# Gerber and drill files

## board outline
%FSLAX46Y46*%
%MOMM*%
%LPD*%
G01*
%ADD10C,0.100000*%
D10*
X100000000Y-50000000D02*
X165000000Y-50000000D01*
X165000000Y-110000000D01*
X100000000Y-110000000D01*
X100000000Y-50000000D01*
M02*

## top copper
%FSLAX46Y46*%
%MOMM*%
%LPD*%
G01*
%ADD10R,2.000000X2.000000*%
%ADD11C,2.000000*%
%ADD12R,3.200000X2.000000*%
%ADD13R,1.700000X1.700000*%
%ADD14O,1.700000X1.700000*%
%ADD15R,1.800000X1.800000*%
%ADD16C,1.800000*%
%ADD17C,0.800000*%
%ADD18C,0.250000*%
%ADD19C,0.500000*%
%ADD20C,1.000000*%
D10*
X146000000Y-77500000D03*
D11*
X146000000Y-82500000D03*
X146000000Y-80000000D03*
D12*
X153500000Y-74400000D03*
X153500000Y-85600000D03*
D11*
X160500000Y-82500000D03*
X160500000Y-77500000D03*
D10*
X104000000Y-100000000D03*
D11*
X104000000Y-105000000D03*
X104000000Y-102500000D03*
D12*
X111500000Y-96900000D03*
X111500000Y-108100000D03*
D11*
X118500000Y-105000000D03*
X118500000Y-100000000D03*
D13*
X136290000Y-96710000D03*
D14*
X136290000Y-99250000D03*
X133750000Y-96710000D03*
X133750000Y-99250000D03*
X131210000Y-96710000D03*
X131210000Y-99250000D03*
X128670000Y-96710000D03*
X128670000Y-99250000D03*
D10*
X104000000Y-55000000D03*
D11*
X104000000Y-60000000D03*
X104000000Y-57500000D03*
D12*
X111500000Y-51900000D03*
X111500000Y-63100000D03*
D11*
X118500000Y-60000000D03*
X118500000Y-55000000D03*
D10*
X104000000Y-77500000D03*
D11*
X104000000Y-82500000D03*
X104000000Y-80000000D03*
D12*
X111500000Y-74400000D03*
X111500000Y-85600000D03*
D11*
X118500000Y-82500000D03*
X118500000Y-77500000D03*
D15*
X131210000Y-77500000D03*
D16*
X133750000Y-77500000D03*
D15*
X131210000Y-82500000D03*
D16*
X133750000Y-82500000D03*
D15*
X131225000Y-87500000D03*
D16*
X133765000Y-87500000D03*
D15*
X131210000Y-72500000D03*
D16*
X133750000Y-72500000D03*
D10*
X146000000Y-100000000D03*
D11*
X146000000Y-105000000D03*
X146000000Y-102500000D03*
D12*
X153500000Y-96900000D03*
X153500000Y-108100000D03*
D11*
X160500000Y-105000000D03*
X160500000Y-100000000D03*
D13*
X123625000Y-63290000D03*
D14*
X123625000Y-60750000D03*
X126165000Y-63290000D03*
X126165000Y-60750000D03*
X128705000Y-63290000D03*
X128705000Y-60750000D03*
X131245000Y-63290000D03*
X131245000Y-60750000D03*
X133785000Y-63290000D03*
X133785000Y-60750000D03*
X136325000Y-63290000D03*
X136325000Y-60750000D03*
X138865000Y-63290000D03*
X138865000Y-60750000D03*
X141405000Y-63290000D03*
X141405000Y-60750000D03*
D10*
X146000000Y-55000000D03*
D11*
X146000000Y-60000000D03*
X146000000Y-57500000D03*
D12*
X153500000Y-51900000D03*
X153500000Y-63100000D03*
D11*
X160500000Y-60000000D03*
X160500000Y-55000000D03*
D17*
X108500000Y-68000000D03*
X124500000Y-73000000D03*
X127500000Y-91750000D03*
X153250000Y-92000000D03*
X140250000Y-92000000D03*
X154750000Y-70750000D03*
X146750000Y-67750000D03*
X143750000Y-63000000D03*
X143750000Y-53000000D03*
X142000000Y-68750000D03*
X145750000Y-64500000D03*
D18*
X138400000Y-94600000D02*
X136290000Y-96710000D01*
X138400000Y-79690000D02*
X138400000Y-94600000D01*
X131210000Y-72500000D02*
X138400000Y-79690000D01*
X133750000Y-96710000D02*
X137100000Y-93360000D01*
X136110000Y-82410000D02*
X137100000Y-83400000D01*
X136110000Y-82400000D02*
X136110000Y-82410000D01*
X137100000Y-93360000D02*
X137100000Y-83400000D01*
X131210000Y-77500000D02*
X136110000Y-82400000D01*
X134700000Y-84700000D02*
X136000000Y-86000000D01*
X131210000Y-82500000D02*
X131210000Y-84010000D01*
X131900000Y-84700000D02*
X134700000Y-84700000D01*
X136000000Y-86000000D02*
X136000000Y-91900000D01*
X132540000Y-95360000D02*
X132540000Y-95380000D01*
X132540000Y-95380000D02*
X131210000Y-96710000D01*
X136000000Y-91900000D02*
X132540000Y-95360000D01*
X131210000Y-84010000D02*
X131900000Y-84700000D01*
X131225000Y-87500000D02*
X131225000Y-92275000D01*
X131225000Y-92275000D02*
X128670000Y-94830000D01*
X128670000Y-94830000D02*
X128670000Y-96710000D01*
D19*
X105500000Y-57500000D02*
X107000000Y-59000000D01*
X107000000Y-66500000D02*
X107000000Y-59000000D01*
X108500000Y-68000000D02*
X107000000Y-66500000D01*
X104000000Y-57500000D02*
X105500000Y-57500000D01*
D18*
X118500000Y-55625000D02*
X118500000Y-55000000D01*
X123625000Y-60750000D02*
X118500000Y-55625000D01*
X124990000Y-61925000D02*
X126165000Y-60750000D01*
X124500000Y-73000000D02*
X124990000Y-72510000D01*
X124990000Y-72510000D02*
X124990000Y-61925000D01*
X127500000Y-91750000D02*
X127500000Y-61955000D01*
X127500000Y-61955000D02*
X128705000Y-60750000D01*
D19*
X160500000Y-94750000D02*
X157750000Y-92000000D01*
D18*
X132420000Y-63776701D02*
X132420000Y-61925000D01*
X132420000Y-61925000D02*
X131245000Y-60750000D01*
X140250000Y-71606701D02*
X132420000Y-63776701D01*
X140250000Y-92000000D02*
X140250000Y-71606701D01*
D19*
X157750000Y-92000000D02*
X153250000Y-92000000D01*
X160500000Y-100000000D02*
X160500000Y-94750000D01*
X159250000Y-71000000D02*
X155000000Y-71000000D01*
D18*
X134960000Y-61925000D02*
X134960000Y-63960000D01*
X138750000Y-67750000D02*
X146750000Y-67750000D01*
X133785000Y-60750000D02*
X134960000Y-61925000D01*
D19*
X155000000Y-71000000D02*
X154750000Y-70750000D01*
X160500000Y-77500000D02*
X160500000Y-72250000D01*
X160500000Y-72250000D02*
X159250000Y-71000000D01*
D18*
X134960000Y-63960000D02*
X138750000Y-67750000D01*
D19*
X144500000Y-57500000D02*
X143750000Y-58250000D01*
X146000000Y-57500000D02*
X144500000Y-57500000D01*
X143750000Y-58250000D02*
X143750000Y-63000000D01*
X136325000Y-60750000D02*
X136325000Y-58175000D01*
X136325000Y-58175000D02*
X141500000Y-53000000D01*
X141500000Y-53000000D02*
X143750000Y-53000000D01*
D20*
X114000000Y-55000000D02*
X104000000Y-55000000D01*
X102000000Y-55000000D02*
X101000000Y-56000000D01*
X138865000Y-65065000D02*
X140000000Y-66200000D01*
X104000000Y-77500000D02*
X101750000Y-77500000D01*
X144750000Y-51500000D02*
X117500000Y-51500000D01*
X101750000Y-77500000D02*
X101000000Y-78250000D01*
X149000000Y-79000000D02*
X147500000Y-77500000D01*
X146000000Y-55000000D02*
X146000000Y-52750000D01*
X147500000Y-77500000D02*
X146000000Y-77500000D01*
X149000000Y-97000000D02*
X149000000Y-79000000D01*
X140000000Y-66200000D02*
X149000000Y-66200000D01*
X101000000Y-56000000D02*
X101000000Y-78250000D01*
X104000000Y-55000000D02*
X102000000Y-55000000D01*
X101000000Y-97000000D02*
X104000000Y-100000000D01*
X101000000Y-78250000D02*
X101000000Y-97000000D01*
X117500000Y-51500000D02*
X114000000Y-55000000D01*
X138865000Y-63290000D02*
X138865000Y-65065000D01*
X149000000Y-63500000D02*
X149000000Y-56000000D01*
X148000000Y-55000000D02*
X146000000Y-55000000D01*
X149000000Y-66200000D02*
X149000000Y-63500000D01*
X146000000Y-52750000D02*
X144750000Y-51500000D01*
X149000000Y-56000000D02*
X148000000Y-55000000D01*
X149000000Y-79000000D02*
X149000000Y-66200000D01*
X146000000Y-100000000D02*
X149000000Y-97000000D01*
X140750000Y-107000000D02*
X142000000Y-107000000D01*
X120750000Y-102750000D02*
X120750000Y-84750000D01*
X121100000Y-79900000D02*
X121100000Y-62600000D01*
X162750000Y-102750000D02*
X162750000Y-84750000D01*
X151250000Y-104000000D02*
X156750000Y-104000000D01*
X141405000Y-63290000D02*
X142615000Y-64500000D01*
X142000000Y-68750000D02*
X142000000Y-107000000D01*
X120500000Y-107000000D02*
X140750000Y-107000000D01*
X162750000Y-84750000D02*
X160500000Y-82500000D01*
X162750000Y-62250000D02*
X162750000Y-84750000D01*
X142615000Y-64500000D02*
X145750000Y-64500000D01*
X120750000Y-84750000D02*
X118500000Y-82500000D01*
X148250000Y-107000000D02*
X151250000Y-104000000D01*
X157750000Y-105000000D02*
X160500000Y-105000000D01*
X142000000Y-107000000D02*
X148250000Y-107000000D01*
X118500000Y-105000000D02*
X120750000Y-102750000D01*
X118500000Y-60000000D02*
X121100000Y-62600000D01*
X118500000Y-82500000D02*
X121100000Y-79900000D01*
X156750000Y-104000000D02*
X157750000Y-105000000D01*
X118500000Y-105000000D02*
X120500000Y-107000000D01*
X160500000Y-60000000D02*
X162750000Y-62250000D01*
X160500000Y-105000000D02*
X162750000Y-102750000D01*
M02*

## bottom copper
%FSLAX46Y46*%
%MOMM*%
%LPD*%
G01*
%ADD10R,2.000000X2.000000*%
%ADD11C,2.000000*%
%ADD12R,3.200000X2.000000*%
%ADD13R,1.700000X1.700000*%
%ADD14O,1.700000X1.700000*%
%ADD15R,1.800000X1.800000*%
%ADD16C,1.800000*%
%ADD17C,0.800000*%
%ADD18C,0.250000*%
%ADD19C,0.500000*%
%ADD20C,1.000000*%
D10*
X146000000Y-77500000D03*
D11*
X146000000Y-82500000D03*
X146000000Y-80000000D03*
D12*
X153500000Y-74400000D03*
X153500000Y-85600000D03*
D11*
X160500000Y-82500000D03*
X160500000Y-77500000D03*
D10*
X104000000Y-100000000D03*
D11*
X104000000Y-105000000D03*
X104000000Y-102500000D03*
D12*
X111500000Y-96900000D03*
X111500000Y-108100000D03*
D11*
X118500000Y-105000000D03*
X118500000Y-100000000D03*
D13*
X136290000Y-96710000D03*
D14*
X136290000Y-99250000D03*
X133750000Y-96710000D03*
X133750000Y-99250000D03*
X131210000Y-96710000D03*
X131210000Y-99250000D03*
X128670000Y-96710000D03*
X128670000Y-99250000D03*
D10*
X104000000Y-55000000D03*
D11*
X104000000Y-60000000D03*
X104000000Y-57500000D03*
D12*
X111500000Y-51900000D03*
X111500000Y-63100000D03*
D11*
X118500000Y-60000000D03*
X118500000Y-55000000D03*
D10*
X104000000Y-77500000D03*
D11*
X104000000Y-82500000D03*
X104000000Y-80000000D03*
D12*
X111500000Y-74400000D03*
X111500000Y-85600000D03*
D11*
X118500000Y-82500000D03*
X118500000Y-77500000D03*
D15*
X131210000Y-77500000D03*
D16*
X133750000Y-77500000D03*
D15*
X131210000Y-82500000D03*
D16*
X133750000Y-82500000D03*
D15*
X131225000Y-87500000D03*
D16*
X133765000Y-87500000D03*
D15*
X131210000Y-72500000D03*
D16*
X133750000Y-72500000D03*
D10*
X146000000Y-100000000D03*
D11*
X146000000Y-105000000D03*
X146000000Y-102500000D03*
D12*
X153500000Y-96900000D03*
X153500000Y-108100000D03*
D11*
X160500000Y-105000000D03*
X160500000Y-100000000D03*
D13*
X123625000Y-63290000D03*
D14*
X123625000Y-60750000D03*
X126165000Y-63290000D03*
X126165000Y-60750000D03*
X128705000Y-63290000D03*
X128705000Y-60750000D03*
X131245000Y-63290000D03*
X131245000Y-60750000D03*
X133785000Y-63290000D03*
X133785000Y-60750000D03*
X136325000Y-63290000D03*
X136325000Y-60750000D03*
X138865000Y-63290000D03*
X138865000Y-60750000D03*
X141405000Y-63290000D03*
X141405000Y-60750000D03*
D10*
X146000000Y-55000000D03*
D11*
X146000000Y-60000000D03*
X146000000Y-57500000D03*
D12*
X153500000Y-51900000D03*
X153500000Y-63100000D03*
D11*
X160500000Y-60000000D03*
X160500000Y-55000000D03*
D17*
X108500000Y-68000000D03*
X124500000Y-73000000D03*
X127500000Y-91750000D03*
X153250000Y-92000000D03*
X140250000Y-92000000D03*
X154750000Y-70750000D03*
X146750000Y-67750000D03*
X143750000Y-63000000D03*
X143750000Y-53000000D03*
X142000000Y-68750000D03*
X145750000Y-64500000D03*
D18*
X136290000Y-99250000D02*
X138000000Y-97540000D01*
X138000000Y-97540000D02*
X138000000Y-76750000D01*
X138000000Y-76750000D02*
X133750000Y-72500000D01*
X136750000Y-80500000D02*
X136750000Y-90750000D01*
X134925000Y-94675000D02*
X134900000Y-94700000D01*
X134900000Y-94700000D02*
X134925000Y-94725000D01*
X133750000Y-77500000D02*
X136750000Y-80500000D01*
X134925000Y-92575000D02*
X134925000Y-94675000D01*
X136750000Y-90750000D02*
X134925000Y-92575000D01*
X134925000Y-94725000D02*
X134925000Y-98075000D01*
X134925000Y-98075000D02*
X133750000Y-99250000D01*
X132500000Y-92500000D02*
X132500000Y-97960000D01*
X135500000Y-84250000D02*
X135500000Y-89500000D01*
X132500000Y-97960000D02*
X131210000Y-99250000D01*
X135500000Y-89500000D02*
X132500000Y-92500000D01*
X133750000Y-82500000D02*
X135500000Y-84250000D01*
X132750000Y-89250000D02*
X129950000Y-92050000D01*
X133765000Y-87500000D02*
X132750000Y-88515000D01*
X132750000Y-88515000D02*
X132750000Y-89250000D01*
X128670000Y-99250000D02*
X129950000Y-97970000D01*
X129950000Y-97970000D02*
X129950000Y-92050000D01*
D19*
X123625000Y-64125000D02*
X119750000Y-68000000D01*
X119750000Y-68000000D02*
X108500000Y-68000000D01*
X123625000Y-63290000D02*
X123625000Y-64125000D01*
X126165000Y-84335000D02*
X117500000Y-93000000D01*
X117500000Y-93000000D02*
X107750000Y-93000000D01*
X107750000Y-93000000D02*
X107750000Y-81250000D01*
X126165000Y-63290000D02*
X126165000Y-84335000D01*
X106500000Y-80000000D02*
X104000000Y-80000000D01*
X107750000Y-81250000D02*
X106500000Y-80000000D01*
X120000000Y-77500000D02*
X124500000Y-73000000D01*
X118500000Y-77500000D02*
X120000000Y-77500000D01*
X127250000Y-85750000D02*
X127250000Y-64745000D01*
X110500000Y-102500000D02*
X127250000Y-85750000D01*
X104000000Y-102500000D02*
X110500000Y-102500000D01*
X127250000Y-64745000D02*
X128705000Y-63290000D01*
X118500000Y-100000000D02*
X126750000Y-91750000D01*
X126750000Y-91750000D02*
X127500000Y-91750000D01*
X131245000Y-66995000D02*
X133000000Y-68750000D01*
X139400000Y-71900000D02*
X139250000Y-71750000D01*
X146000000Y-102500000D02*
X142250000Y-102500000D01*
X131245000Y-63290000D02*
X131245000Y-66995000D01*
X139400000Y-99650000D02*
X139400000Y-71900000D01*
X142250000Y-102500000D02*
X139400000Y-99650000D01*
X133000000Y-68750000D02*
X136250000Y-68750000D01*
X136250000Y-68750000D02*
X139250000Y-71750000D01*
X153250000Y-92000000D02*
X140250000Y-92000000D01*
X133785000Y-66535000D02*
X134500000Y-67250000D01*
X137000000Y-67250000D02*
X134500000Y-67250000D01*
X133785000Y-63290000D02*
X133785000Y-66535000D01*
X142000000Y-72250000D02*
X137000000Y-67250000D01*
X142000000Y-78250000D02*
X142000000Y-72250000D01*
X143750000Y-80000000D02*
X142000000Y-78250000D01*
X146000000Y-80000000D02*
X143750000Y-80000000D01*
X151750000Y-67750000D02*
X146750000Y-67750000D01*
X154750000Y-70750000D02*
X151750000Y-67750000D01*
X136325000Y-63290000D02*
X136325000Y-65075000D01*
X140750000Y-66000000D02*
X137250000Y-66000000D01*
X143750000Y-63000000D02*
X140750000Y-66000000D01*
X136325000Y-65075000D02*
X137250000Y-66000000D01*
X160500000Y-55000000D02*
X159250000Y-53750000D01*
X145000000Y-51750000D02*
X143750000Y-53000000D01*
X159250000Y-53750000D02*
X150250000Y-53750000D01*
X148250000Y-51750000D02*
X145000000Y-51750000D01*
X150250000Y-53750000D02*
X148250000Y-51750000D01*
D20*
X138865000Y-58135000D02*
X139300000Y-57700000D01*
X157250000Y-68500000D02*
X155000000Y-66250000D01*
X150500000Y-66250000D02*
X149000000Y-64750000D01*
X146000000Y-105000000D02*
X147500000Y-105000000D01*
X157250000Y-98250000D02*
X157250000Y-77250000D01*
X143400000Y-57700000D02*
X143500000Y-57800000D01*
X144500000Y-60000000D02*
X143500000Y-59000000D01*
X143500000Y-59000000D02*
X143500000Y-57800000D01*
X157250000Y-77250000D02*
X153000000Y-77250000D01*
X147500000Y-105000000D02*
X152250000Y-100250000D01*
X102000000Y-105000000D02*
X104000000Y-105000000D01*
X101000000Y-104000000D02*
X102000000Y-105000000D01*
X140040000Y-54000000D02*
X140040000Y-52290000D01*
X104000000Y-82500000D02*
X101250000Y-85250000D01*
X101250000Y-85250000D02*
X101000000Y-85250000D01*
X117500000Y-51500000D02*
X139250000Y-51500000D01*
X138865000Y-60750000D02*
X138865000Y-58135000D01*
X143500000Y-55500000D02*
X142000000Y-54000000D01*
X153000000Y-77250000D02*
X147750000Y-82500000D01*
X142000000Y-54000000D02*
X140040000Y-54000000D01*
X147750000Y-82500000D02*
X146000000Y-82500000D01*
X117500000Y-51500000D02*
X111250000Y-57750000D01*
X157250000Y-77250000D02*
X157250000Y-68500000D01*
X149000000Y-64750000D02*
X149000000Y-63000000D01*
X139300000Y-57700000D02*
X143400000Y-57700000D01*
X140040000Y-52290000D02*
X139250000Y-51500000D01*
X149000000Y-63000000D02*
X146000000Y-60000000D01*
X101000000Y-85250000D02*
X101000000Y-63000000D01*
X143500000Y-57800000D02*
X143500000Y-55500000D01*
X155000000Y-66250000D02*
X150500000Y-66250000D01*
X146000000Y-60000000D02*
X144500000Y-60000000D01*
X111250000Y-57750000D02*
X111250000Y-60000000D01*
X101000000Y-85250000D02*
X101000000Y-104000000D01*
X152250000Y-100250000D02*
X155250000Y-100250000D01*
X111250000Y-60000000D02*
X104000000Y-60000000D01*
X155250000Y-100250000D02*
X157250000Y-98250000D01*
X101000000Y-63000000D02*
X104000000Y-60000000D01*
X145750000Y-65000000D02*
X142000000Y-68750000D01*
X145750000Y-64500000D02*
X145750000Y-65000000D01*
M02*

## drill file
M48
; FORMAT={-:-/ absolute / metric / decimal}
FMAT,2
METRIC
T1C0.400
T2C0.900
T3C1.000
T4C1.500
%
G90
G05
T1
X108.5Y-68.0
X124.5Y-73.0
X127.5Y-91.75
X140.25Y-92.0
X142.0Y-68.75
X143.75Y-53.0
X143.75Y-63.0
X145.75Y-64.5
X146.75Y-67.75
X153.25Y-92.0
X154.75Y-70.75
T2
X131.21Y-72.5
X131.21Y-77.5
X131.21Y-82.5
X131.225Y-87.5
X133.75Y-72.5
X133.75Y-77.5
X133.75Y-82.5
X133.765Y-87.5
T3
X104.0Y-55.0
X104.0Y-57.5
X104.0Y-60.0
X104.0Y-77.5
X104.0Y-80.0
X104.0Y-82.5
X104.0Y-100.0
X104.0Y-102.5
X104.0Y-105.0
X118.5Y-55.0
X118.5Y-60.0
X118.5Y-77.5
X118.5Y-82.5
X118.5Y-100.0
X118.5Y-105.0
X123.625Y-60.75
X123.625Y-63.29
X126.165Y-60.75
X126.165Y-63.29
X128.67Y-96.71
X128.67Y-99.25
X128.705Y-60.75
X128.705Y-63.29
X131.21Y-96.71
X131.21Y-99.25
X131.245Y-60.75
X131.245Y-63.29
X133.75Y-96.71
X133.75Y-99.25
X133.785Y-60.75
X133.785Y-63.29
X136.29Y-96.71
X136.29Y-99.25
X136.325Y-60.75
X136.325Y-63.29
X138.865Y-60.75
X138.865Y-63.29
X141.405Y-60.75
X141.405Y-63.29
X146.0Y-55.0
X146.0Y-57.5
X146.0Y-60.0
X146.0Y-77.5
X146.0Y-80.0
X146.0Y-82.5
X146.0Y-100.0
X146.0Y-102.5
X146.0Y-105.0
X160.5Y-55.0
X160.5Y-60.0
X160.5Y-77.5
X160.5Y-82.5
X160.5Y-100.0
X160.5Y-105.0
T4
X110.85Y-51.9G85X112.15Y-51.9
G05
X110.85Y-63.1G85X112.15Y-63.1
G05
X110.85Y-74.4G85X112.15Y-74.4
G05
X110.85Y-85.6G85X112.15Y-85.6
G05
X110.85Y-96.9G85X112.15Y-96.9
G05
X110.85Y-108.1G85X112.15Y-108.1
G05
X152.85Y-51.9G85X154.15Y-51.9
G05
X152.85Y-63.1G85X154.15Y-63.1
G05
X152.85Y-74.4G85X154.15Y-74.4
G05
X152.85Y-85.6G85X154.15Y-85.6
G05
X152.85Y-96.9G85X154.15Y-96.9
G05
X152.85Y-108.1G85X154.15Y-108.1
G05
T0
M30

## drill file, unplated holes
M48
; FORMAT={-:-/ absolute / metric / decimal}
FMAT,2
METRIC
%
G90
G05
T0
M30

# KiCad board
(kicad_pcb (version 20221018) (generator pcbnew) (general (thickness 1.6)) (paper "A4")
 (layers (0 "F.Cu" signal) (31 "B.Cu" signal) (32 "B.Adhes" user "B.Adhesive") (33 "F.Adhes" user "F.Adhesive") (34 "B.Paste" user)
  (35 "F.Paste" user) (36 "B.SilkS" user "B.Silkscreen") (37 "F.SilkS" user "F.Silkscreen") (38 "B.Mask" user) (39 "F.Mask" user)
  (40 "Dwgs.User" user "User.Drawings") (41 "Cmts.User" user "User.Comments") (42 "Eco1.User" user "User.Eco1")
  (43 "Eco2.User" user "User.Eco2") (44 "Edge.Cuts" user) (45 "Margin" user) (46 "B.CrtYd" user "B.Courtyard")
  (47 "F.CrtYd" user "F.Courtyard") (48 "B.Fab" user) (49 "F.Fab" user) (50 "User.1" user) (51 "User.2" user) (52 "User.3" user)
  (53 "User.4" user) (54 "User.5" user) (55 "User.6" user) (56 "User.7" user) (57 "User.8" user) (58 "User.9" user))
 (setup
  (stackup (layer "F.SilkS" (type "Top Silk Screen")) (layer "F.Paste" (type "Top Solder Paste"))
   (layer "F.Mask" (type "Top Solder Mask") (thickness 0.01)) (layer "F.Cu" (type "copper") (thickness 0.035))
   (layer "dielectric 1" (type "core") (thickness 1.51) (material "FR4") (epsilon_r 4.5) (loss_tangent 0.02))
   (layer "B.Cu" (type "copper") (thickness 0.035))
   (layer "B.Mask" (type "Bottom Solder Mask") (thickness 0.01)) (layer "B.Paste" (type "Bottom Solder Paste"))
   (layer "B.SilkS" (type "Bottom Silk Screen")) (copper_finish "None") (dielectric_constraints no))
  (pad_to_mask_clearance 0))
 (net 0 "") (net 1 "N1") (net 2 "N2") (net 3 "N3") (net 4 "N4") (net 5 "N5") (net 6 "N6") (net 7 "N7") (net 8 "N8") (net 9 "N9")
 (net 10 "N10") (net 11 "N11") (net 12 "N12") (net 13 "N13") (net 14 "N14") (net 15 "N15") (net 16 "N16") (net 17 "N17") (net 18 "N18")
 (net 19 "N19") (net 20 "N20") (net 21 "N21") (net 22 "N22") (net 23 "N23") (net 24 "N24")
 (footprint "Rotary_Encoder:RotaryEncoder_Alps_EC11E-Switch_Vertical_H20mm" (layer "F.Cu") (at 146 77.5)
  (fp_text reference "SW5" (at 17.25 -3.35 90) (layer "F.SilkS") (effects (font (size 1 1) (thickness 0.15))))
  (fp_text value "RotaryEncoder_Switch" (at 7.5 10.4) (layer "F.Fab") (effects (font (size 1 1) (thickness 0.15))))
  (pad "A" thru_hole rect (at 0 0) (size 2 2) (drill 1) (layers "*.Cu" "*.Mask") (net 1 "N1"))
  (pad "B" thru_hole circle (at 0 5) (size 2 2) (drill 1) (layers "*.Cu" "*.Mask") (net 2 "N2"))
  (pad "C" thru_hole circle (at 0 2.5) (size 2 2) (drill 1) (layers "*.Cu" "*.Mask") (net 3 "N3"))
  (pad "MP" thru_hole rect (at 7.5 -3.1) (size 3.2 2) (drill oval 2.8 1.5) (layers "*.Cu" "*.Mask"))
  (pad "MP" thru_hole rect (at 7.5 8.1) (size 3.2 2) (drill oval 2.8 1.5) (layers "*.Cu" "*.Mask"))
  (pad "S1" thru_hole circle (at 14.5 5) (size 2 2) (drill 1) (layers "*.Cu" "*.Mask") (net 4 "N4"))
  (pad "S2" thru_hole circle (at 14.5 0) (size 2 2) (drill 1) (layers "*.Cu" "*.Mask") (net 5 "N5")))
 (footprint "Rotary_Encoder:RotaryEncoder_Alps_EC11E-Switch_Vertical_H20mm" (layer "F.Cu") (at 104 100)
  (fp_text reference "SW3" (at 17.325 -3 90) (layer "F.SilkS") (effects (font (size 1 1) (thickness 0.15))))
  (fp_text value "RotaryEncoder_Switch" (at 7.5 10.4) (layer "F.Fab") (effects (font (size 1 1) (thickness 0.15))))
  (pad "A" thru_hole rect (at 0 0) (size 2 2) (drill 1) (layers "*.Cu" "*.Mask") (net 1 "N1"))
  (pad "B" thru_hole circle (at 0 5) (size 2 2) (drill 1) (layers "*.Cu" "*.Mask") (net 2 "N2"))
  (pad "C" thru_hole circle (at 0 2.5) (size 2 2) (drill 1) (layers "*.Cu" "*.Mask") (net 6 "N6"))
  (pad "MP" thru_hole rect (at 7.5 -3.1) (size 3.2 2) (drill oval 2.8 1.5) (layers "*.Cu" "*.Mask"))
  (pad "MP" thru_hole rect (at 7.5 8.1) (size 3.2 2) (drill oval 2.8 1.5) (layers "*.Cu" "*.Mask"))
  (pad "S1" thru_hole circle (at 14.5 5) (size 2 2) (drill 1) (layers "*.Cu" "*.Mask") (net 4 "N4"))
  (pad "S2" thru_hole circle (at 14.5 0) (size 2 2) (drill 1) (layers "*.Cu" "*.Mask") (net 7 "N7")))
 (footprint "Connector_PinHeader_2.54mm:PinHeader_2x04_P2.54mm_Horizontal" (layer "F.Cu") (at 136.29 96.71 -90)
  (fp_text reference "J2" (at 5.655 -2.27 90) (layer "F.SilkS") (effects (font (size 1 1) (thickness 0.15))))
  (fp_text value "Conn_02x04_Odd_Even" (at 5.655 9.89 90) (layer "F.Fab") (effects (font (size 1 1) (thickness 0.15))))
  (pad "1" thru_hole rect (at 0 0 270) (size 1.7 1.7) (drill 1) (layers "*.Cu" "*.Mask") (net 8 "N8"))
  (pad "2" thru_hole oval (at 2.54 0 270) (size 1.7 1.7) (drill 1) (layers "*.Cu" "*.Mask") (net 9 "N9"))
  (pad "3" thru_hole oval (at 0 2.54 270) (size 1.7 1.7) (drill 1) (layers "*.Cu" "*.Mask") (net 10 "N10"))
  (pad "4" thru_hole oval (at 2.54 2.54 270) (size 1.7 1.7) (drill 1) (layers "*.Cu" "*.Mask") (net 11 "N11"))
  (pad "5" thru_hole oval (at 0 5.08 270) (size 1.7 1.7) (drill 1) (layers "*.Cu" "*.Mask") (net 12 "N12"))
  (pad "6" thru_hole oval (at 2.54 5.08 270) (size 1.7 1.7) (drill 1) (layers "*.Cu" "*.Mask") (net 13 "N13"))
  (pad "7" thru_hole oval (at 0 7.62 270) (size 1.7 1.7) (drill 1) (layers "*.Cu" "*.Mask") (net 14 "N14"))
  (pad "8" thru_hole oval (at 2.54 7.62 270) (size 1.7 1.7) (drill 1) (layers "*.Cu" "*.Mask") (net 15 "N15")))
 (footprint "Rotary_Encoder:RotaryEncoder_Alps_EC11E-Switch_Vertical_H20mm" (layer "F.Cu") (at 104 55)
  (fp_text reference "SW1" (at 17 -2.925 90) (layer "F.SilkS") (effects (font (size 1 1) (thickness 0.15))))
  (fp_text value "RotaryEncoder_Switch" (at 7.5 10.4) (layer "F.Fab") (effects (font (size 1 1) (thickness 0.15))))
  (pad "A" thru_hole rect (at 0 0) (size 2 2) (drill 1) (layers "*.Cu" "*.Mask") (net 1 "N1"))
  (pad "B" thru_hole circle (at 0 5) (size 2 2) (drill 1) (layers "*.Cu" "*.Mask") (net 2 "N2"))
  (pad "C" thru_hole circle (at 0 2.5) (size 2 2) (drill 1) (layers "*.Cu" "*.Mask") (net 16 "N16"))
  (pad "MP" thru_hole rect (at 7.5 -3.1) (size 3.2 2) (drill oval 2.8 1.5) (layers "*.Cu" "*.Mask"))
  (pad "MP" thru_hole rect (at 7.5 8.1) (size 3.2 2) (drill oval 2.8 1.5) (layers "*.Cu" "*.Mask"))
  (pad "S1" thru_hole circle (at 14.5 5) (size 2 2) (drill 1) (layers "*.Cu" "*.Mask") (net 4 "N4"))
  (pad "S2" thru_hole circle (at 14.5 0) (size 2 2) (drill 1) (layers "*.Cu" "*.Mask") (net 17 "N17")))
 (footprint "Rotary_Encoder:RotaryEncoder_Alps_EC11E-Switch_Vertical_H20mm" (layer "F.Cu") (at 104 77.5)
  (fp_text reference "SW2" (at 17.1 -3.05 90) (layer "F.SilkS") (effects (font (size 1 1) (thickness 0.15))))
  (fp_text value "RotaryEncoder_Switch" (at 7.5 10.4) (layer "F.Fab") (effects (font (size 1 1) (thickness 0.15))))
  (pad "A" thru_hole rect (at 0 0) (size 2 2) (drill 1) (layers "*.Cu" "*.Mask") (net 1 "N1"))
  (pad "B" thru_hole circle (at 0 5) (size 2 2) (drill 1) (layers "*.Cu" "*.Mask") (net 2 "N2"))
  (pad "C" thru_hole circle (at 0 2.5) (size 2 2) (drill 1) (layers "*.Cu" "*.Mask") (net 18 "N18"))
  (pad "MP" thru_hole rect (at 7.5 -3.1) (size 3.2 2) (drill oval 2.8 1.5) (layers "*.Cu" "*.Mask"))
  (pad "MP" thru_hole rect (at 7.5 8.1) (size 3.2 2) (drill oval 2.8 1.5) (layers "*.Cu" "*.Mask"))
  (pad "S1" thru_hole circle (at 14.5 5) (size 2 2) (drill 1) (layers "*.Cu" "*.Mask") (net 4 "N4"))
  (pad "S2" thru_hole circle (at 14.5 0) (size 2 2) (drill 1) (layers "*.Cu" "*.Mask") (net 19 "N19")))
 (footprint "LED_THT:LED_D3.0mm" (layer "F.Cu") (at 131.21 77.5)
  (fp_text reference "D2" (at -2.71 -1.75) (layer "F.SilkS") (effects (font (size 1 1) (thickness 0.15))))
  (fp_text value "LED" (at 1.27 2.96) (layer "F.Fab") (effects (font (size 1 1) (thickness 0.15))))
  (pad "1" thru_hole rect (at 0 0) (size 1.8 1.8) (drill 0.9) (layers "*.Cu" "*.Mask") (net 10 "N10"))
  (pad "2" thru_hole circle (at 2.54 0) (size 1.8 1.8) (drill 0.9) (layers "*.Cu" "*.Mask") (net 11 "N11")))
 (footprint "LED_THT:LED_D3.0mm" (layer "F.Cu") (at 131.21 82.5)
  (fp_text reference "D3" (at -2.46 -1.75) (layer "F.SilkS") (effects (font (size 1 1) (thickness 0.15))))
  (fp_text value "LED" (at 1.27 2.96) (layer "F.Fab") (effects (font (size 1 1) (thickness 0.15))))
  (pad "1" thru_hole rect (at 0 0) (size 1.8 1.8) (drill 0.9) (layers "*.Cu" "*.Mask") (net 12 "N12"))
  (pad "2" thru_hole circle (at 2.54 0) (size 1.8 1.8) (drill 0.9) (layers "*.Cu" "*.Mask") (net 13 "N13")))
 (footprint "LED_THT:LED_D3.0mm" (layer "F.Cu") (at 131.225 87.5)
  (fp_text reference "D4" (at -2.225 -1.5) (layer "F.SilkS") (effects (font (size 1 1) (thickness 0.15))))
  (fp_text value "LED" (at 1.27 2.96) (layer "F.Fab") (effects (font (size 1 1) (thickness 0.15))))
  (pad "1" thru_hole rect (at 0 0) (size 1.8 1.8) (drill 0.9) (layers "*.Cu" "*.Mask") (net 14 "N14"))
  (pad "2" thru_hole circle (at 2.54 0) (size 1.8 1.8) (drill 0.9) (layers "*.Cu" "*.Mask") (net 15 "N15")))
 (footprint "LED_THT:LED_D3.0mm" (layer "F.Cu") (at 131.21 72.5)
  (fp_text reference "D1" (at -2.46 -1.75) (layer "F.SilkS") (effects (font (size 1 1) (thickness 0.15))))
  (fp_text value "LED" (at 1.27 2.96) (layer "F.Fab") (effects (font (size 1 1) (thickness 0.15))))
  (pad "1" thru_hole rect (at 0 0) (size 1.8 1.8) (drill 0.9) (layers "*.Cu" "*.Mask") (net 8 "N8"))
  (pad "2" thru_hole circle (at 2.54 0) (size 1.8 1.8) (drill 0.9) (layers "*.Cu" "*.Mask") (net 9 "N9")))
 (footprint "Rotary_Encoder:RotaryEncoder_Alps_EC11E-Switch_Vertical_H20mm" (layer "F.Cu") (at 146 100)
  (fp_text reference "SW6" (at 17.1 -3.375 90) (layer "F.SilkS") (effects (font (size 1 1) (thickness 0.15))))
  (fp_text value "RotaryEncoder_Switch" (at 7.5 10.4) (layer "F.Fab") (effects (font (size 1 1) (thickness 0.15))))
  (pad "A" thru_hole rect (at 0 0) (size 2 2) (drill 1) (layers "*.Cu" "*.Mask") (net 1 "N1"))
  (pad "B" thru_hole circle (at 0 5) (size 2 2) (drill 1) (layers "*.Cu" "*.Mask") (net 2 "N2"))
  (pad "C" thru_hole circle (at 0 2.5) (size 2 2) (drill 1) (layers "*.Cu" "*.Mask") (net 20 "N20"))
  (pad "MP" thru_hole rect (at 7.5 -3.1) (size 3.2 2) (drill oval 2.8 1.5) (layers "*.Cu" "*.Mask"))
  (pad "MP" thru_hole rect (at 7.5 8.1) (size 3.2 2) (drill oval 2.8 1.5) (layers "*.Cu" "*.Mask"))
  (pad "S1" thru_hole circle (at 14.5 5) (size 2 2) (drill 1) (layers "*.Cu" "*.Mask") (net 4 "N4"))
  (pad "S2" thru_hole circle (at 14.5 0) (size 2 2) (drill 1) (layers "*.Cu" "*.Mask") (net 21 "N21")))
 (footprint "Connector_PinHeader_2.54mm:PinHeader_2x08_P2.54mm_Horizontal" (layer "F.Cu") (at 123.625 63.29 90)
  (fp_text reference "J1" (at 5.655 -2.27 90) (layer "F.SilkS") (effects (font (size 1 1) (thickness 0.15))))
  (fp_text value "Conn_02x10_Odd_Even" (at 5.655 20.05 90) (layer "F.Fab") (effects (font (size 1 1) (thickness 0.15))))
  (pad "1" thru_hole rect (at 0 0 90) (size 1.7 1.7) (drill 1) (layers "*.Cu" "*.Mask") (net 16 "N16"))
  (pad "2" thru_hole oval (at 2.54 0 90) (size 1.7 1.7) (drill 1) (layers "*.Cu" "*.Mask") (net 17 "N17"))
  (pad "3" thru_hole oval (at 0 2.54 90) (size 1.7 1.7) (drill 1) (layers "*.Cu" "*.Mask") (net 18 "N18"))
  (pad "4" thru_hole oval (at 2.54 2.54 90) (size 1.7 1.7) (drill 1) (layers "*.Cu" "*.Mask") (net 19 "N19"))
  (pad "5" thru_hole oval (at 0 5.08 90) (size 1.7 1.7) (drill 1) (layers "*.Cu" "*.Mask") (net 6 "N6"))
  (pad "6" thru_hole oval (at 2.54 5.08 90) (size 1.7 1.7) (drill 1) (layers "*.Cu" "*.Mask") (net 7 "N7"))
  (pad "7" thru_hole oval (at 0 7.62 90) (size 1.7 1.7) (drill 1) (layers "*.Cu" "*.Mask") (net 20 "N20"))
  (pad "8" thru_hole oval (at 2.54 7.62 90) (size 1.7 1.7) (drill 1) (layers "*.Cu" "*.Mask") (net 21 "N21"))
  (pad "9" thru_hole oval (at 0 10.16 90) (size 1.7 1.7) (drill 1) (layers "*.Cu" "*.Mask") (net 3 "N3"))
  (pad "10" thru_hole oval (at 2.54 10.16 90) (size 1.7 1.7) (drill 1) (layers "*.Cu" "*.Mask") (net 5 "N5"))
  (pad "11" thru_hole oval (at 0 12.7 90) (size 1.7 1.7) (drill 1) (layers "*.Cu" "*.Mask") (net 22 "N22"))
  (pad "12" thru_hole oval (at 2.54 12.7 90) (size 1.7 1.7) (drill 1) (layers "*.Cu" "*.Mask") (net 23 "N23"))
  (pad "13" thru_hole oval (at 0 15.24 90) (size 1.7 1.7) (drill 1) (layers "*.Cu" "*.Mask") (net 1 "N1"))
  (pad "14" thru_hole oval (at 2.54 15.24 90) (size 1.7 1.7) (drill 1) (layers "*.Cu" "*.Mask") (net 2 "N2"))
  (pad "15" thru_hole oval (at 0 17.78 90) (size 1.7 1.7) (drill 1) (layers "*.Cu" "*.Mask") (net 4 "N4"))
  (pad "16" thru_hole oval (at 2.54 17.78 90) (size 1.7 1.7) (drill 1) (layers "*.Cu" "*.Mask") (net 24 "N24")))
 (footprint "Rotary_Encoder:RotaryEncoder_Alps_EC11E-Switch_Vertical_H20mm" (layer "F.Cu") (at 146 55)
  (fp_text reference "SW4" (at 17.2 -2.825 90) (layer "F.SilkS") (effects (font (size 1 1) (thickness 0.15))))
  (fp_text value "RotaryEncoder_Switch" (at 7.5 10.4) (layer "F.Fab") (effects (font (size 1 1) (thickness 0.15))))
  (pad "A" thru_hole rect (at 0 0) (size 2 2) (drill 1) (layers "*.Cu" "*.Mask") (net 1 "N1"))
  (pad "B" thru_hole circle (at 0 5) (size 2 2) (drill 1) (layers "*.Cu" "*.Mask") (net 2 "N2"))
  (pad "C" thru_hole circle (at 0 2.5) (size 2 2) (drill 1) (layers "*.Cu" "*.Mask") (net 22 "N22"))
  (pad "MP" thru_hole rect (at 7.5 -3.1) (size 3.2 2) (drill oval 2.8 1.5) (layers "*.Cu" "*.Mask"))
  (pad "MP" thru_hole rect (at 7.5 8.1) (size 3.2 2) (drill oval 2.8 1.5) (layers "*.Cu" "*.Mask"))
  (pad "S1" thru_hole circle (at 14.5 5) (size 2 2) (drill 1) (layers "*.Cu" "*.Mask") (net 4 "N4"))
  (pad "S2" thru_hole circle (at 14.5 0) (size 2 2) (drill 1) (layers "*.Cu" "*.Mask") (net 23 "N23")))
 (gr_rect (start 100 50) (end 165 110) (stroke (width 0.1) (type default)) (fill none) (layer "Edge.Cuts"))
 (segment (start 138.4 94.6) (end 136.29 96.71) (width 0.25) (layer "F.Cu") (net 8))
 (segment (start 138.4 79.69) (end 138.4 94.6) (width 0.25) (layer "F.Cu") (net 8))
 (segment (start 131.21 72.5) (end 138.4 79.69) (width 0.25) (layer "F.Cu") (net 8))
 (segment (start 136.29 99.25) (end 138 97.54) (width 0.25) (layer "B.Cu") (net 9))
 (segment (start 138 97.54) (end 138 76.75) (width 0.25) (layer "B.Cu") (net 9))
 (segment (start 138 76.75) (end 133.75 72.5) (width 0.25) (layer "B.Cu") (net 9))
 (segment (start 133.75 96.71) (end 137.1 93.36) (width 0.25) (layer "F.Cu") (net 10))
 (segment (start 136.11 82.41) (end 137.1 83.4) (width 0.25) (layer "F.Cu") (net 10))
 (segment (start 136.11 82.4) (end 136.11 82.41) (width 0.25) (layer "F.Cu") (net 10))
 (segment (start 137.1 93.36) (end 137.1 83.4) (width 0.25) (layer "F.Cu") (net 10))
 (segment (start 131.21 77.5) (end 136.11 82.4) (width 0.25) (layer "F.Cu") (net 10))
 (segment (start 136.75 80.5) (end 136.75 90.75) (width 0.25) (layer "B.Cu") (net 11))
 (segment (start 134.925 94.675) (end 134.9 94.7) (width 0.25) (layer "B.Cu") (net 11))
 (segment (start 134.9 94.7) (end 134.925 94.725) (width 0.25) (layer "B.Cu") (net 11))
 (segment (start 133.75 77.5) (end 136.75 80.5) (width 0.25) (layer "B.Cu") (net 11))
 (segment (start 134.925 92.575) (end 134.925 94.675) (width 0.25) (layer "B.Cu") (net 11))
 (segment (start 136.75 90.75) (end 134.925 92.575) (width 0.25) (layer "B.Cu") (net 11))
 (segment (start 134.925 94.725) (end 134.925 98.075) (width 0.25) (layer "B.Cu") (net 11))
 (segment (start 134.925 98.075) (end 133.75 99.25) (width 0.25) (layer "B.Cu") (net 11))
 (segment (start 134.7 84.7) (end 136 86) (width 0.25) (layer "F.Cu") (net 12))
 (segment (start 131.21 82.5) (end 131.21 84.01) (width 0.25) (layer "F.Cu") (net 12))
 (segment (start 131.9 84.7) (end 134.7 84.7) (width 0.25) (layer "F.Cu") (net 12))
 (segment (start 136 86) (end 136 91.9) (width 0.25) (layer "F.Cu") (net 12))
 (segment (start 132.54 95.36) (end 132.54 95.38) (width 0.25) (layer "F.Cu") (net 12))
 (segment (start 132.54 95.38) (end 131.21 96.71) (width 0.25) (layer "F.Cu") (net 12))
 (segment (start 136 91.9) (end 132.54 95.36) (width 0.25) (layer "F.Cu") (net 12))
 (segment (start 131.21 84.01) (end 131.9 84.7) (width 0.25) (layer "F.Cu") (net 12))
 (segment (start 132.5 92.5) (end 132.5 97.96) (width 0.25) (layer "B.Cu") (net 13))
 (segment (start 135.5 84.25) (end 135.5 89.5) (width 0.25) (layer "B.Cu") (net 13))
 (segment (start 132.5 97.96) (end 131.21 99.25) (width 0.25) (layer "B.Cu") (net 13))
 (segment (start 135.5 89.5) (end 132.5 92.5) (width 0.25) (layer "B.Cu") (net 13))
 (segment (start 133.75 82.5) (end 135.5 84.25) (width 0.25) (layer "B.Cu") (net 13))
 (segment (start 131.225 87.5) (end 131.225 92.275) (width 0.25) (layer "F.Cu") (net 14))
 (segment (start 131.225 92.275) (end 128.67 94.83) (width 0.25) (layer "F.Cu") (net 14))
 (segment (start 128.67 94.83) (end 128.67 96.71) (width 0.25) (layer "F.Cu") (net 14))
 (segment (start 132.75 89.25) (end 129.95 92.05) (width 0.25) (layer "B.Cu") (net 15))
 (segment (start 133.765 87.5) (end 132.75 88.515) (width 0.25) (layer "B.Cu") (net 15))
 (segment (start 132.75 88.515) (end 132.75 89.25) (width 0.25) (layer "B.Cu") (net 15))
 (segment (start 128.67 99.25) (end 129.95 97.97) (width 0.25) (layer "B.Cu") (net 15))
 (segment (start 129.95 97.97) (end 129.95 92.05) (width 0.25) (layer "B.Cu") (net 15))
 (segment (start 105.5 57.5) (end 107 59) (width 0.5) (layer "F.Cu") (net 16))
 (segment (start 107 66.5) (end 107 59) (width 0.5) (layer "F.Cu") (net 16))
 (segment (start 108.5 68) (end 107 66.5) (width 0.5) (layer "F.Cu") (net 16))
 (segment (start 104 57.5) (end 105.5 57.5) (width 0.5) (layer "F.Cu") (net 16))
 (via (at 108.5 68) (size 0.8) (drill 0.4) (layers "F.Cu" "B.Cu") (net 16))
 (segment (start 123.625 64.125) (end 119.75 68) (width 0.5) (layer "B.Cu") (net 16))
 (segment (start 119.75 68) (end 108.5 68) (width 0.5) (layer "B.Cu") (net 16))
 (segment (start 123.625 63.29) (end 123.625 64.125) (width 0.5) (layer "B.Cu") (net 16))
 (segment (start 118.5 55.625) (end 118.5 55) (width 0.25) (layer "F.Cu") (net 17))
 (segment (start 123.625 60.75) (end 118.5 55.625) (width 0.25) (layer "F.Cu") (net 17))
 (segment (start 126.165 84.335) (end 117.5 93) (width 0.5) (layer "B.Cu") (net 18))
 (segment (start 117.5 93) (end 107.75 93) (width 0.5) (layer "B.Cu") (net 18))
 (segment (start 107.75 93) (end 107.75 81.25) (width 0.5) (layer "B.Cu") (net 18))
 (segment (start 126.165 63.29) (end 126.165 84.335) (width 0.5) (layer "B.Cu") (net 18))
 (segment (start 106.5 80) (end 104 80) (width 0.5) (layer "B.Cu") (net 18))
 (segment (start 107.75 81.25) (end 106.5 80) (width 0.5) (layer "B.Cu") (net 18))
 (segment (start 124.99 61.925) (end 126.165 60.75) (width 0.25) (layer "F.Cu") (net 19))
 (segment (start 124.5 73) (end 124.99 72.51) (width 0.25) (layer "F.Cu") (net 19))
 (segment (start 124.99 72.51) (end 124.99 61.925) (width 0.25) (layer "F.Cu") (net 19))
 (via (at 124.5 73) (size 0.8) (drill 0.4) (layers "F.Cu" "B.Cu") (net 19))
 (segment (start 120 77.5) (end 124.5 73) (width 0.5) (layer "B.Cu") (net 19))
 (segment (start 118.5 77.5) (end 120 77.5) (width 0.5) (layer "B.Cu") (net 19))
 (segment (start 127.25 85.75) (end 127.25 64.745) (width 0.5) (layer "B.Cu") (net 6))
 (segment (start 110.5 102.5) (end 127.25 85.75) (width 0.5) (layer "B.Cu") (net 6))
 (segment (start 104 102.5) (end 110.5 102.5) (width 0.5) (layer "B.Cu") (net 6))
 (segment (start 127.25 64.745) (end 128.705 63.29) (width 0.5) (layer "B.Cu") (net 6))
 (segment (start 127.5 91.75) (end 127.5 61.955) (width 0.25) (layer "F.Cu") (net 7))
 (segment (start 127.5 61.955) (end 128.705 60.75) (width 0.25) (layer "F.Cu") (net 7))
 (via (at 127.5 91.75) (size 0.8) (drill 0.4) (layers "F.Cu" "B.Cu") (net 7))
 (segment (start 118.5 100) (end 126.75 91.75) (width 0.5) (layer "B.Cu") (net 7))
 (segment (start 126.75 91.75) (end 127.5 91.75) (width 0.5) (layer "B.Cu") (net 7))
 (segment (start 131.245 66.995) (end 133 68.75) (width 0.5) (layer "B.Cu") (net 20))
 (segment (start 139.4 71.9) (end 139.25 71.75) (width 0.5) (layer "B.Cu") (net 20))
 (segment (start 146 102.5) (end 142.25 102.5) (width 0.5) (layer "B.Cu") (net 20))
 (segment (start 131.245 63.29) (end 131.245 66.995) (width 0.5) (layer "B.Cu") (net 20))
 (segment (start 139.4 99.65) (end 139.4 71.9) (width 0.5) (layer "B.Cu") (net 20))
 (segment (start 142.25 102.5) (end 139.4 99.65) (width 0.5) (layer "B.Cu") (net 20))
 (segment (start 133 68.75) (end 136.25 68.75) (width 0.5) (layer "B.Cu") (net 20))
 (segment (start 136.25 68.75) (end 139.25 71.75) (width 0.5) (layer "B.Cu") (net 20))
 (segment (start 160.5 94.75) (end 157.75 92) (width 0.5) (layer "F.Cu") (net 21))
 (segment (start 132.42 63.776701) (end 132.42 61.925) (width 0.25) (layer "F.Cu") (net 21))
 (segment (start 132.42 61.925) (end 131.245 60.75) (width 0.25) (layer "F.Cu") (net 21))
 (segment (start 140.25 71.606701) (end 132.42 63.776701) (width 0.25) (layer "F.Cu") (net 21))
 (segment (start 140.25 92) (end 140.25 71.606701) (width 0.25) (layer "F.Cu") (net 21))
 (segment (start 157.75 92) (end 153.25 92) (width 0.5) (layer "F.Cu") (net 21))
 (segment (start 160.5 100) (end 160.5 94.75) (width 0.5) (layer "F.Cu") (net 21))
 (via (at 153.25 92) (size 0.8) (drill 0.4) (layers "F.Cu" "B.Cu") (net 21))
 (via (at 140.25 92) (size 0.8) (drill 0.4) (layers "F.Cu" "B.Cu") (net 21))
 (segment (start 153.25 92) (end 140.25 92) (width 0.5) (layer "B.Cu") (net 21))
 (segment (start 133.785 66.535) (end 134.5 67.25) (width 0.5) (layer "B.Cu") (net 3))
 (segment (start 137 67.25) (end 134.5 67.25) (width 0.5) (layer "B.Cu") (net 3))
 (segment (start 133.785 63.29) (end 133.785 66.535) (width 0.5) (layer "B.Cu") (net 3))
 (segment (start 142 72.25) (end 137 67.25) (width 0.5) (layer "B.Cu") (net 3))
 (segment (start 142 78.25) (end 142 72.25) (width 0.5) (layer "B.Cu") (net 3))
 (segment (start 143.75 80) (end 142 78.25) (width 0.5) (layer "B.Cu") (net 3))
 (segment (start 146 80) (end 143.75 80) (width 0.5) (layer "B.Cu") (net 3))
 (segment (start 159.25 71) (end 155 71) (width 0.5) (layer "F.Cu") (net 5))
 (segment (start 134.96 61.925) (end 134.96 63.96) (width 0.25) (layer "F.Cu") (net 5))
 (segment (start 138.75 67.75) (end 146.75 67.75) (width 0.25) (layer "F.Cu") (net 5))
 (segment (start 133.785 60.75) (end 134.96 61.925) (width 0.25) (layer "F.Cu") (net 5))
 (segment (start 155 71) (end 154.75 70.75) (width 0.5) (layer "F.Cu") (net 5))
 (segment (start 160.5 77.5) (end 160.5 72.25) (width 0.5) (layer "F.Cu") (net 5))
 (segment (start 160.5 72.25) (end 159.25 71) (width 0.5) (layer "F.Cu") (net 5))
 (segment (start 134.96 63.96) (end 138.75 67.75) (width 0.25) (layer "F.Cu") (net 5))
 (via (at 154.75 70.75) (size 0.8) (drill 0.4) (layers "F.Cu" "B.Cu") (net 5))
 (via (at 146.75 67.75) (size 0.8) (drill 0.4) (layers "F.Cu" "B.Cu") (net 5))
 (segment (start 151.75 67.75) (end 146.75 67.75) (width 0.5) (layer "B.Cu") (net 5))
 (segment (start 154.75 70.75) (end 151.75 67.75) (width 0.5) (layer "B.Cu") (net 5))
 (segment (start 144.5 57.5) (end 143.75 58.25) (width 0.5) (layer "F.Cu") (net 22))
 (segment (start 146 57.5) (end 144.5 57.5) (width 0.5) (layer "F.Cu") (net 22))
 (segment (start 143.75 58.25) (end 143.75 63) (width 0.5) (layer "F.Cu") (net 22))
 (via (at 143.75 63) (size 0.8) (drill 0.4) (layers "F.Cu" "B.Cu") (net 22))
 (segment (start 136.325 63.29) (end 136.325 65.075) (width 0.5) (layer "B.Cu") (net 22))
 (segment (start 140.75 66) (end 137.25 66) (width 0.5) (layer "B.Cu") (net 22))
 (segment (start 143.75 63) (end 140.75 66) (width 0.5) (layer "B.Cu") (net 22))
 (segment (start 136.325 65.075) (end 137.25 66) (width 0.5) (layer "B.Cu") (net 22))
 (segment (start 136.325 60.75) (end 136.325 58.175) (width 0.5) (layer "F.Cu") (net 23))
 (segment (start 136.325 58.175) (end 141.5 53) (width 0.5) (layer "F.Cu") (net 23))
 (segment (start 141.5 53) (end 143.75 53) (width 0.5) (layer "F.Cu") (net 23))
 (via (at 143.75 53) (size 0.8) (drill 0.4) (layers "F.Cu" "B.Cu") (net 23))
 (segment (start 160.5 55) (end 159.25 53.75) (width 0.5) (layer "B.Cu") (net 23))
 (segment (start 145 51.75) (end 143.75 53) (width 0.5) (layer "B.Cu") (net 23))
 (segment (start 159.25 53.75) (end 150.25 53.75) (width 0.5) (layer "B.Cu") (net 23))
 (segment (start 148.25 51.75) (end 145 51.75) (width 0.5) (layer "B.Cu") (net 23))
 (segment (start 150.25 53.75) (end 148.25 51.75) (width 0.5) (layer "B.Cu") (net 23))
 (segment (start 114 55) (end 104 55) (width 1) (layer "F.Cu") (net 1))
 (segment (start 102 55) (end 101 56) (width 1) (layer "F.Cu") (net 1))
 (segment (start 138.865 65.065) (end 140 66.2) (width 1) (layer "F.Cu") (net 1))
 (segment (start 104 77.5) (end 101.75 77.5) (width 1) (layer "F.Cu") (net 1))
 (segment (start 144.75 51.5) (end 117.5 51.5) (width 1) (layer "F.Cu") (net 1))
 (segment (start 101.75 77.5) (end 101 78.25) (width 1) (layer "F.Cu") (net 1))
 (segment (start 149 79) (end 147.5 77.5) (width 1) (layer "F.Cu") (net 1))
 (segment (start 146 55) (end 146 52.75) (width 1) (layer "F.Cu") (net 1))
 (segment (start 147.5 77.5) (end 146 77.5) (width 1) (layer "F.Cu") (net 1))
 (segment (start 149 97) (end 149 79) (width 1) (layer "F.Cu") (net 1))
 (segment (start 140 66.2) (end 149 66.2) (width 1) (layer "F.Cu") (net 1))
 (segment (start 101 56) (end 101 78.25) (width 1) (layer "F.Cu") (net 1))
 (segment (start 104 55) (end 102 55) (width 1) (layer "F.Cu") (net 1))
 (segment (start 101 97) (end 104 100) (width 1) (layer "F.Cu") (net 1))
 (segment (start 101 78.25) (end 101 97) (width 1) (layer "F.Cu") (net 1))
 (segment (start 117.5 51.5) (end 114 55) (width 1) (layer "F.Cu") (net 1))
 (segment (start 138.865 63.29) (end 138.865 65.065) (width 1) (layer "F.Cu") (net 1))
 (segment (start 149 63.5) (end 149 56) (width 1) (layer "F.Cu") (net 1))
 (segment (start 148 55) (end 146 55) (width 1) (layer "F.Cu") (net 1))
 (segment (start 149 66.2) (end 149 63.5) (width 1) (layer "F.Cu") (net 1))
 (segment (start 146 52.75) (end 144.75 51.5) (width 1) (layer "F.Cu") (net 1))
 (segment (start 149 56) (end 148 55) (width 1) (layer "F.Cu") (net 1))
 (segment (start 149 79) (end 149 66.2) (width 1) (layer "F.Cu") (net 1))
 (segment (start 146 100) (end 149 97) (width 1) (layer "F.Cu") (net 1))
 (segment (start 138.865 58.135) (end 139.3 57.7) (width 1) (layer "B.Cu") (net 2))
 (segment (start 157.25 68.5) (end 155 66.25) (width 1) (layer "B.Cu") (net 2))
 (segment (start 150.5 66.25) (end 149 64.75) (width 1) (layer "B.Cu") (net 2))
 (segment (start 146 105) (end 147.5 105) (width 1) (layer "B.Cu") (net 2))
 (segment (start 157.25 98.25) (end 157.25 77.25) (width 1) (layer "B.Cu") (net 2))
 (segment (start 143.4 57.7) (end 143.5 57.8) (width 1) (layer "B.Cu") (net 2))
 (segment (start 144.5 60) (end 143.5 59) (width 1) (layer "B.Cu") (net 2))
 (segment (start 143.5 59) (end 143.5 57.8) (width 1) (layer "B.Cu") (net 2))
 (segment (start 157.25 77.25) (end 153 77.25) (width 1) (layer "B.Cu") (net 2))
 (segment (start 147.5 105) (end 152.25 100.25) (width 1) (layer "B.Cu") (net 2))
 (segment (start 102 105) (end 104 105) (width 1) (layer "B.Cu") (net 2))
 (segment (start 101 104) (end 102 105) (width 1) (layer "B.Cu") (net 2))
 (segment (start 140.04 54) (end 140.04 52.29) (width 1) (layer "B.Cu") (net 2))
 (segment (start 104 82.5) (end 101.25 85.25) (width 1) (layer "B.Cu") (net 2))
 (segment (start 101.25 85.25) (end 101 85.25) (width 1) (layer "B.Cu") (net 2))
 (segment (start 117.5 51.5) (end 139.25 51.5) (width 1) (layer "B.Cu") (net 2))
 (segment (start 138.865 60.75) (end 138.865 58.135) (width 1) (layer "B.Cu") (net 2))
 (segment (start 143.5 55.5) (end 142 54) (width 1) (layer "B.Cu") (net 2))
 (segment (start 153 77.25) (end 147.75 82.5) (width 1) (layer "B.Cu") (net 2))
 (segment (start 142 54) (end 140.04 54) (width 1) (layer "B.Cu") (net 2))
 (segment (start 147.75 82.5) (end 146 82.5) (width 1) (layer "B.Cu") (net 2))
 (segment (start 117.5 51.5) (end 111.25 57.75) (width 1) (layer "B.Cu") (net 2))
 (segment (start 157.25 77.25) (end 157.25 68.5) (width 1) (layer "B.Cu") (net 2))
 (segment (start 149 64.75) (end 149 63) (width 1) (layer "B.Cu") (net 2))
 (segment (start 139.3 57.7) (end 143.4 57.7) (width 1) (layer "B.Cu") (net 2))
 (segment (start 140.04 52.29) (end 139.25 51.5) (width 1) (layer "B.Cu") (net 2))
 (segment (start 149 63) (end 146 60) (width 1) (layer "B.Cu") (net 2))
 (segment (start 101 85.25) (end 101 63) (width 1) (layer "B.Cu") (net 2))
 (segment (start 143.5 57.8) (end 143.5 55.5) (width 1) (layer "B.Cu") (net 2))
 (segment (start 155 66.25) (end 150.5 66.25) (width 1) (layer "B.Cu") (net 2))
 (segment (start 146 60) (end 144.5 60) (width 1) (layer "B.Cu") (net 2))
 (segment (start 111.25 57.75) (end 111.25 60) (width 1) (layer "B.Cu") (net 2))
 (segment (start 101 85.25) (end 101 104) (width 1) (layer "B.Cu") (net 2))
 (segment (start 152.25 100.25) (end 155.25 100.25) (width 1) (layer "B.Cu") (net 2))
 (segment (start 111.25 60) (end 104 60) (width 1) (layer "B.Cu") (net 2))
 (segment (start 155.25 100.25) (end 157.25 98.25) (width 1) (layer "B.Cu") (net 2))
 (segment (start 101 63) (end 104 60) (width 1) (layer "B.Cu") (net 2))
 (segment (start 140.75 107) (end 142 107) (width 1) (layer "F.Cu") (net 4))
 (segment (start 120.75 102.75) (end 120.75 84.75) (width 1) (layer "F.Cu") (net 4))
 (segment (start 121.1 79.9) (end 121.1 62.6) (width 1) (layer "F.Cu") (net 4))
 (segment (start 162.75 102.75) (end 162.75 84.75) (width 1) (layer "F.Cu") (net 4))
 (segment (start 151.25 104) (end 156.75 104) (width 1) (layer "F.Cu") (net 4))
 (segment (start 141.405 63.29) (end 142.615 64.5) (width 1) (layer "F.Cu") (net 4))
 (segment (start 142 68.75) (end 142 107) (width 1) (layer "F.Cu") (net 4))
 (segment (start 120.5 107) (end 140.75 107) (width 1) (layer "F.Cu") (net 4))
 (segment (start 162.75 84.75) (end 160.5 82.5) (width 1) (layer "F.Cu") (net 4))
 (segment (start 162.75 62.25) (end 162.75 84.75) (width 1) (layer "F.Cu") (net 4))
 (segment (start 142.615 64.5) (end 145.75 64.5) (width 1) (layer "F.Cu") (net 4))
 (segment (start 120.75 84.75) (end 118.5 82.5) (width 1) (layer "F.Cu") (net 4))
 (segment (start 148.25 107) (end 151.25 104) (width 1) (layer "F.Cu") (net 4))
 (segment (start 157.75 105) (end 160.5 105) (width 1) (layer "F.Cu") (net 4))
 (segment (start 142 107) (end 148.25 107) (width 1) (layer "F.Cu") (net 4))
 (segment (start 118.5 105) (end 120.75 102.75) (width 1) (layer "F.Cu") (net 4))
 (segment (start 118.5 60) (end 121.1 62.6) (width 1) (layer "F.Cu") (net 4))
 (segment (start 118.5 82.5) (end 121.1 79.9) (width 1) (layer "F.Cu") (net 4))
 (segment (start 156.75 104) (end 157.75 105) (width 1) (layer "F.Cu") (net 4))
 (segment (start 118.5 105) (end 120.5 107) (width 1) (layer "F.Cu") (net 4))
 (segment (start 160.5 60) (end 162.75 62.25) (width 1) (layer "F.Cu") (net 4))
 (segment (start 160.5 105) (end 162.75 102.75) (width 1) (layer "F.Cu") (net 4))
 (via (at 142 68.75) (size 0.8) (drill 0.4) (layers "F.Cu" "B.Cu") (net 4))
 (via (at 145.75 64.5) (size 0.8) (drill 0.4) (layers "F.Cu" "B.Cu") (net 4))
 (segment (start 145.75 65) (end 142 68.75) (width 1) (layer "B.Cu") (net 4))
 (segment (start 145.75 64.5) (end 145.75 65) (width 1) (layer "B.Cu") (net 4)))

